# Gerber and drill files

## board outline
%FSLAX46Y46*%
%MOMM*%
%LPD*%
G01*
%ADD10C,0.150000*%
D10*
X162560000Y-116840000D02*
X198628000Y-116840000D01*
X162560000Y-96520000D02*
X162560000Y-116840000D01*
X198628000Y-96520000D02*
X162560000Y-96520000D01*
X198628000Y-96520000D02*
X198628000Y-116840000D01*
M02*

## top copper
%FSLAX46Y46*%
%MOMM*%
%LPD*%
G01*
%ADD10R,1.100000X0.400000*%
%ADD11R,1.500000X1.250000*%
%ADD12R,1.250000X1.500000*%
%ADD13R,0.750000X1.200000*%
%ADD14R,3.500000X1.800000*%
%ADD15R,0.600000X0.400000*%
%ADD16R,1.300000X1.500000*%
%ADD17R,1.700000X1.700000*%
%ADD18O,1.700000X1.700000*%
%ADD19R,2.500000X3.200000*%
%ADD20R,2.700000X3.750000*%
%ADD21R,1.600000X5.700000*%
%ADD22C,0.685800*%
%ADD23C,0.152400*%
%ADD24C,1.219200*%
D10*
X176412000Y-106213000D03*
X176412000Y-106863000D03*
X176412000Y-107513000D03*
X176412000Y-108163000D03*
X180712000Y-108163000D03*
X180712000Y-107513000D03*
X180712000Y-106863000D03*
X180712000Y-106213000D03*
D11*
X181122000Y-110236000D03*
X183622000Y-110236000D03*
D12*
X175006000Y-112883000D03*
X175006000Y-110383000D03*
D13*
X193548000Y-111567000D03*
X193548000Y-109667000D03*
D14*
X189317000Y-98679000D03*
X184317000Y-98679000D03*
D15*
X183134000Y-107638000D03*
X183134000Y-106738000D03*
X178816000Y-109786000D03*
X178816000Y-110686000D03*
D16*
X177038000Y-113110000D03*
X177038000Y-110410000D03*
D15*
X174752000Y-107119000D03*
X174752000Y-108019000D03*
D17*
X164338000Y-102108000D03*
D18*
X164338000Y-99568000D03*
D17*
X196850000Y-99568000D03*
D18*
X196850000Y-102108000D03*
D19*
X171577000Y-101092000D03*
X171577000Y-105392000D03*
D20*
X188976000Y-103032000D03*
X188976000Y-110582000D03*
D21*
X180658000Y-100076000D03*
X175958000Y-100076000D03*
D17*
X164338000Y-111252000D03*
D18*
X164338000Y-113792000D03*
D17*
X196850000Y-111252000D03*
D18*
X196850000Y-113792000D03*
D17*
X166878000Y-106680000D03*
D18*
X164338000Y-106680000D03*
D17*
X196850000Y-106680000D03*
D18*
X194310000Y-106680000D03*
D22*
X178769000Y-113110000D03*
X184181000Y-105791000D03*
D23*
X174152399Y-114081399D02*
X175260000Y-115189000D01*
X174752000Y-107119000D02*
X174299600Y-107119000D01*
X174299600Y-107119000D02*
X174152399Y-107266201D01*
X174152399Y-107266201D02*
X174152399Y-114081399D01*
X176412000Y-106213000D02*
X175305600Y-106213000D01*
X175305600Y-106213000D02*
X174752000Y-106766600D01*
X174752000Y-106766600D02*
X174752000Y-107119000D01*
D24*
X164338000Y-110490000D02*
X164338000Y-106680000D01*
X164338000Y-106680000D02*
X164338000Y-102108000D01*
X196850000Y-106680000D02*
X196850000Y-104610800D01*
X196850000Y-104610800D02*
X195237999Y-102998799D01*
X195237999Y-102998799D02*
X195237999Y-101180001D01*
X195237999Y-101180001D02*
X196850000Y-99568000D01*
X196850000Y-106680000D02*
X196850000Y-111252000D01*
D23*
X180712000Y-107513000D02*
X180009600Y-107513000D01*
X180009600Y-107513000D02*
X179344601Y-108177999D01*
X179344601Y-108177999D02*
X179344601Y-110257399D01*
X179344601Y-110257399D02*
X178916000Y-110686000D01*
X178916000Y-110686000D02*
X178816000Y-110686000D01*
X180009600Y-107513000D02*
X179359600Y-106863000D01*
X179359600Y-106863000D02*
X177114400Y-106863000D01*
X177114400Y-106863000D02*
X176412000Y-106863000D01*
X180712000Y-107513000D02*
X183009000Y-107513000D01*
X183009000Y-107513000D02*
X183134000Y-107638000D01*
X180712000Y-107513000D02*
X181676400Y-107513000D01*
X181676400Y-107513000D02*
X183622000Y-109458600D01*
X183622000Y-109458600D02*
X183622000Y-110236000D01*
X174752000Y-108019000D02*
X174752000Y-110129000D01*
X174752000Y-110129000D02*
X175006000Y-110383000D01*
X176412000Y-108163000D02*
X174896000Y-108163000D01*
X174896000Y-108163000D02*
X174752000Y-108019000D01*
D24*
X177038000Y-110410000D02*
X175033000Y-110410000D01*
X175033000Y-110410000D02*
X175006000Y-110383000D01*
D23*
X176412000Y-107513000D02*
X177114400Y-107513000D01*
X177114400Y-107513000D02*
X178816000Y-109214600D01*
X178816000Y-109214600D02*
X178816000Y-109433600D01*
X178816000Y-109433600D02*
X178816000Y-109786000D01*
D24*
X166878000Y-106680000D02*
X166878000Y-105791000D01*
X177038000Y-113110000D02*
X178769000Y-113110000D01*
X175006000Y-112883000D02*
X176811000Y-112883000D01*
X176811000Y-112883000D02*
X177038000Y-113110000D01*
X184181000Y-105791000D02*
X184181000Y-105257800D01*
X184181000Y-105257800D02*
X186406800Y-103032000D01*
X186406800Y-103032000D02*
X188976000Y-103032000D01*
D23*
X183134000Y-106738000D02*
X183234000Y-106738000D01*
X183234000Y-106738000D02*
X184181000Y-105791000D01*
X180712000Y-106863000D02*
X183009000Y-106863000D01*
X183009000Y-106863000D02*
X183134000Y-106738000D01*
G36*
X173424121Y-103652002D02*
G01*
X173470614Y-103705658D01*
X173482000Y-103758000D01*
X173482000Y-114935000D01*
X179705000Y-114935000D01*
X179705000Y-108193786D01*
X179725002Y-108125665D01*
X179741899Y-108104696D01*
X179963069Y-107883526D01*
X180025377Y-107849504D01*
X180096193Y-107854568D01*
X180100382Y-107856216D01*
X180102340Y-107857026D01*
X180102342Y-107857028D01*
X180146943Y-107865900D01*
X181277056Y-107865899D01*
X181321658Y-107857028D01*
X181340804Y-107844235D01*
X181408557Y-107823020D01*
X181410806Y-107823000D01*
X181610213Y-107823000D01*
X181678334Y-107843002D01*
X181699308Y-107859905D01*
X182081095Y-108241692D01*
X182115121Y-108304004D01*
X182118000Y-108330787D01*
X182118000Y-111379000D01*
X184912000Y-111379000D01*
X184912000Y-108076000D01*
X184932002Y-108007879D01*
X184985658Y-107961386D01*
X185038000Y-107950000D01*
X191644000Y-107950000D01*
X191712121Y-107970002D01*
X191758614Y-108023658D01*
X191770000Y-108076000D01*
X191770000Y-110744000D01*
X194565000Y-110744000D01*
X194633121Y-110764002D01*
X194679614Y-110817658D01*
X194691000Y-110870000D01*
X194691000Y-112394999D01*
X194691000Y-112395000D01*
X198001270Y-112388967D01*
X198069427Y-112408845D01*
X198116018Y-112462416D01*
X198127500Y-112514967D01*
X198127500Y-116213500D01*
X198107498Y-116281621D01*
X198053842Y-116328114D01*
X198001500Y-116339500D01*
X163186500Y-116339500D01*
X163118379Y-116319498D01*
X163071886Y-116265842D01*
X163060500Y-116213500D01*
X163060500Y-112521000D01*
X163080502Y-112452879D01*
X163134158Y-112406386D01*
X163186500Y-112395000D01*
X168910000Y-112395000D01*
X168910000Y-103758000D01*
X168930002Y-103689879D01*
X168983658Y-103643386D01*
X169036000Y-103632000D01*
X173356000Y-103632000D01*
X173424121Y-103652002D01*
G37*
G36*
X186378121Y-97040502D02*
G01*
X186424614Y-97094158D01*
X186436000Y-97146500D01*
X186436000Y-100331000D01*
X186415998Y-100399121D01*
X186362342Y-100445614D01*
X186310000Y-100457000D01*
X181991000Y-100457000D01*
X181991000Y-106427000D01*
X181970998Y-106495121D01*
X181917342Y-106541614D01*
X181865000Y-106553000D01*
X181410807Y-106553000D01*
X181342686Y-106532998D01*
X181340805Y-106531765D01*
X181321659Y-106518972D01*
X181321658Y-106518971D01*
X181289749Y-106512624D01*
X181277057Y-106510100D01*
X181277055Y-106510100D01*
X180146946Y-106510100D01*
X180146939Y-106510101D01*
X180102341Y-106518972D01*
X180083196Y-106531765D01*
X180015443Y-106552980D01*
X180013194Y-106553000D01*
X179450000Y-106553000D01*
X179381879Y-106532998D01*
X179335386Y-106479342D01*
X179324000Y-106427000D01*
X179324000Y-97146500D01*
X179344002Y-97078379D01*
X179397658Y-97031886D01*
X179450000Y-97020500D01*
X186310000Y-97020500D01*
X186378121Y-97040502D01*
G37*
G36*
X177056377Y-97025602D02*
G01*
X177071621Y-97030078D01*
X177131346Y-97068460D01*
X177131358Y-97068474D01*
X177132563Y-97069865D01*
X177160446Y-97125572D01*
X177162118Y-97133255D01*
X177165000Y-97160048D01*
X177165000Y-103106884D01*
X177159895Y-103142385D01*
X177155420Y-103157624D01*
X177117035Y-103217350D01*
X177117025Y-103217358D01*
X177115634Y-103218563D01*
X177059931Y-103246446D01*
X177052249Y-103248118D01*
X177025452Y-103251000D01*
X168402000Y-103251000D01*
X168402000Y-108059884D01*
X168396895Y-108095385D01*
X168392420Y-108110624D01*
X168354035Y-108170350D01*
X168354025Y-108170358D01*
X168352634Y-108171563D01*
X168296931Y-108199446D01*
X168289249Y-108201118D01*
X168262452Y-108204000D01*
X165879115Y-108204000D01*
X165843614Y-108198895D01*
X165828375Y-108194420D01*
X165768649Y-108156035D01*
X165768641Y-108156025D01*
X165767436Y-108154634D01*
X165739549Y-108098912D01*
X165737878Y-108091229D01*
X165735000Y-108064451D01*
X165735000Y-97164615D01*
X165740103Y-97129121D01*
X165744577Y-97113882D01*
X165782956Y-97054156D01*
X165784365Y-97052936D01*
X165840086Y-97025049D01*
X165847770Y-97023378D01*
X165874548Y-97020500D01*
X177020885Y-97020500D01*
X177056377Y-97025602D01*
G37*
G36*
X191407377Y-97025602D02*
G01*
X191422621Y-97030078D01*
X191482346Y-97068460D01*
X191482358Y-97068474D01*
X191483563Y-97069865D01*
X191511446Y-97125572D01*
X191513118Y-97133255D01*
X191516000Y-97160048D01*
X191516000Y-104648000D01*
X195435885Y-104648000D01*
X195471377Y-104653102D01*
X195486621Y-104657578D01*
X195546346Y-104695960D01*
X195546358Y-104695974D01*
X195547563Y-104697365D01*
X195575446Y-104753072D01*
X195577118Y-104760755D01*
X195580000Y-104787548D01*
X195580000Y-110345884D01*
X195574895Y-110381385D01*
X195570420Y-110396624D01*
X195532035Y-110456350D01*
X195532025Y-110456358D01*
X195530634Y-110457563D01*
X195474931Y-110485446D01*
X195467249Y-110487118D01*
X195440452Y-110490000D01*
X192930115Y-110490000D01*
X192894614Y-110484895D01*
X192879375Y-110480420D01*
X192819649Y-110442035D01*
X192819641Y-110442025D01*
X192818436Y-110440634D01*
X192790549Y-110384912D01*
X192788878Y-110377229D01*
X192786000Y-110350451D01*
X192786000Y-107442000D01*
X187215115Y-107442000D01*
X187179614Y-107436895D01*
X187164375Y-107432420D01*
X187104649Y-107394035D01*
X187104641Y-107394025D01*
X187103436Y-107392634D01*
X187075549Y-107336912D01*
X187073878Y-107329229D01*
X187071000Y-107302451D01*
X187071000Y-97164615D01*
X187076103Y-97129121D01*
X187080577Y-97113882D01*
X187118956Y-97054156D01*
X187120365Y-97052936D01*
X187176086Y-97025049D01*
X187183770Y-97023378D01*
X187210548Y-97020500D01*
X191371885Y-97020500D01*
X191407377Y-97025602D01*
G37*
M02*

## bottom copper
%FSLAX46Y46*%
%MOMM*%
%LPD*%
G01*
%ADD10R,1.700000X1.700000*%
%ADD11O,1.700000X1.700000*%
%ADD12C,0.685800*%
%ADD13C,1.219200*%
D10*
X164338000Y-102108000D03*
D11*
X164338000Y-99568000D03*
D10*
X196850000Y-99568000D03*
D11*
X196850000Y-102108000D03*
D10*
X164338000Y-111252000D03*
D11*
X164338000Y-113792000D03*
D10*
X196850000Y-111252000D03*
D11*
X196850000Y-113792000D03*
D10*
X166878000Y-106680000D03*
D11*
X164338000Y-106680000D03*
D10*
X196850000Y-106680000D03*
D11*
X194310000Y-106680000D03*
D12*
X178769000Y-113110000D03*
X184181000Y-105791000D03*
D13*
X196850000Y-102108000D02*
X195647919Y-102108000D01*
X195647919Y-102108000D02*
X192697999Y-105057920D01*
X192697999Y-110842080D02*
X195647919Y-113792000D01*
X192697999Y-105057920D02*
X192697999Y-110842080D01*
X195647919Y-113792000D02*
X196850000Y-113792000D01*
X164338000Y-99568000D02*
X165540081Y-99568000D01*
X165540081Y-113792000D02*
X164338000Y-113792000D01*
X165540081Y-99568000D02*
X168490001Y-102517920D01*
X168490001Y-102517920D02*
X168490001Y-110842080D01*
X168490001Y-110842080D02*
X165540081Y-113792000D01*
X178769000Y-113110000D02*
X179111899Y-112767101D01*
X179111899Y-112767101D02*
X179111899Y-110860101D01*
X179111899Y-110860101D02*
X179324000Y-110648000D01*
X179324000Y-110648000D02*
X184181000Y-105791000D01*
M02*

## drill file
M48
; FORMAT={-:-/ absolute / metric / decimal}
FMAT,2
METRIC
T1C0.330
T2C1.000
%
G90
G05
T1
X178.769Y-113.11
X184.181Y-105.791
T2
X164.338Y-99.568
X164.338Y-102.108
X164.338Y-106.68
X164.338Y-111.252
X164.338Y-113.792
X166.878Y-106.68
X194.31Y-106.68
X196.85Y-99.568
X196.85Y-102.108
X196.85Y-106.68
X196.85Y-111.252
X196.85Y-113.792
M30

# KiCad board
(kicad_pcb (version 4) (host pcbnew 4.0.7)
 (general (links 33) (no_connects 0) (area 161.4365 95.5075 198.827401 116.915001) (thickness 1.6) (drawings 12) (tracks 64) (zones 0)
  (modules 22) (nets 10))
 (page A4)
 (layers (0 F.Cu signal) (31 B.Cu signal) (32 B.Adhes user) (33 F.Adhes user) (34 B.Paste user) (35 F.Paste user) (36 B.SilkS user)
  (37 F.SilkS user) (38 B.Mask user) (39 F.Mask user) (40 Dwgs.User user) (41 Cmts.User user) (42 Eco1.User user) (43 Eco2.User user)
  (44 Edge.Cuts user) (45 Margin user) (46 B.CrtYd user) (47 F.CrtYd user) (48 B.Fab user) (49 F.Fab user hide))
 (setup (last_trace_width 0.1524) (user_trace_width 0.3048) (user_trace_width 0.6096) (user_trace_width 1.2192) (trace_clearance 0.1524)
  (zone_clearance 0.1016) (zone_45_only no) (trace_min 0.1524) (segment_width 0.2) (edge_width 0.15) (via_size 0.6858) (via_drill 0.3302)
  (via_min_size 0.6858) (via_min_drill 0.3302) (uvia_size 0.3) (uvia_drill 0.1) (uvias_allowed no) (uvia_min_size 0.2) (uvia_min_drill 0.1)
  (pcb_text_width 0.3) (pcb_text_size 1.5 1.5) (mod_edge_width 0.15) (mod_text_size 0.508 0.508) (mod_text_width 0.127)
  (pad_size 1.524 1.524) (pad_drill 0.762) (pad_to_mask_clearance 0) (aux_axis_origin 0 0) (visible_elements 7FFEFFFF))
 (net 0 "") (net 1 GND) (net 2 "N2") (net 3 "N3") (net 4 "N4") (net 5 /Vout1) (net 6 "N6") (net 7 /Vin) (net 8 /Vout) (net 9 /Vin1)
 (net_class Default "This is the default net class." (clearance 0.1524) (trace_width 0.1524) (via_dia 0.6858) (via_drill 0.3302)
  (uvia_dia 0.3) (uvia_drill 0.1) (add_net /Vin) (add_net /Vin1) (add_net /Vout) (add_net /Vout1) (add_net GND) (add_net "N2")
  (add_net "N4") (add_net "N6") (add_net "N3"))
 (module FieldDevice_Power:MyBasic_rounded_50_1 (layer B.Cu) (at 180.848 100.457 180)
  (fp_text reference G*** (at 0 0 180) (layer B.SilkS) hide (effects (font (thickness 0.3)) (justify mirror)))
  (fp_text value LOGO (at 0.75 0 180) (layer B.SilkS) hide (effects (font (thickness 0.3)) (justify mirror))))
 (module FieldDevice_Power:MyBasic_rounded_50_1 (layer F.Cu) (at 170.18 111.633)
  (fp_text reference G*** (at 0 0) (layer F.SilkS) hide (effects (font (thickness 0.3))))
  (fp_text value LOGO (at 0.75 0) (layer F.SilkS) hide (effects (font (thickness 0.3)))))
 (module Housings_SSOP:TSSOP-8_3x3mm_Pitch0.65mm (layer F.Cu) (at 178.562 107.188)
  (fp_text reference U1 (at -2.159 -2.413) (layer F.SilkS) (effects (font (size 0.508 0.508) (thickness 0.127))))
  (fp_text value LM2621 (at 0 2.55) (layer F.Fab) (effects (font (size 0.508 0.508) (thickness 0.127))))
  (pad 1 smd rect (at -2.15 -0.975) (size 1.1 0.4) (layers F.Cu F.Paste F.Mask) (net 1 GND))
  (pad 2 smd rect (at -2.15 -0.325) (size 1.1 0.4) (layers F.Cu F.Paste F.Mask) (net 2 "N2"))
  (pad 3 smd rect (at -2.15 0.325) (size 1.1 0.4) (layers F.Cu F.Paste F.Mask) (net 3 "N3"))
  (pad 4 smd rect (at -2.15 0.975) (size 1.1 0.4) (layers F.Cu F.Paste F.Mask) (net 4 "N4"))
  (pad 5 smd rect (at 2.15 0.975) (size 1.1 0.4) (layers F.Cu F.Paste F.Mask) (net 1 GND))
  (pad 6 smd rect (at 2.15 0.325) (size 1.1 0.4) (layers F.Cu F.Paste F.Mask) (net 2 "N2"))
  (pad 7 smd rect (at 2.15 -0.325) (size 1.1 0.4) (layers F.Cu F.Paste F.Mask) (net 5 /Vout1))
  (pad 8 smd rect (at 2.15 -0.975) (size 1.1 0.4) (layers F.Cu F.Paste F.Mask) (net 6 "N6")))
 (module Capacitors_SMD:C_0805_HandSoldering (layer F.Cu) (at 182.372 110.236)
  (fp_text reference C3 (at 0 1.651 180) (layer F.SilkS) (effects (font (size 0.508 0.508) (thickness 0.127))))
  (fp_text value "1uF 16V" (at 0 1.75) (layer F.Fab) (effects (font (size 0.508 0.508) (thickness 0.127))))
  (pad 1 smd rect (at -1.25 0) (size 1.5 1.25) (layers F.Cu F.Paste F.Mask) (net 1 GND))
  (pad 2 smd rect (at 1.25 0) (size 1.5 1.25) (layers F.Cu F.Paste F.Mask) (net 2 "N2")))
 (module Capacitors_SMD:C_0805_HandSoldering (layer F.Cu) (at 175.006 111.633 90)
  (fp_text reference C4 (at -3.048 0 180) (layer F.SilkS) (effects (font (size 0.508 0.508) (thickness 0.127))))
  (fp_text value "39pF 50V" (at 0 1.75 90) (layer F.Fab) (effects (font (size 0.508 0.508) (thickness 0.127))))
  (pad 1 smd rect (at -1.25 0 90) (size 1.5 1.25) (layers F.Cu F.Paste F.Mask) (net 5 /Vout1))
  (pad 2 smd rect (at 1.25 0 90) (size 1.5 1.25) (layers F.Cu F.Paste F.Mask) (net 4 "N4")))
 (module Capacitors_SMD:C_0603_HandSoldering (layer F.Cu) (at 193.548 110.617 90)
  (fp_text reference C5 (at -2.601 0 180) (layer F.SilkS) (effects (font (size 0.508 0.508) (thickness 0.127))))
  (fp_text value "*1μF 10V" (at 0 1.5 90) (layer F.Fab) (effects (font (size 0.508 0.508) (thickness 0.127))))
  (pad 1 smd rect (at -0.95 0 90) (size 1.2 0.75) (layers F.Cu F.Paste F.Mask) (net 1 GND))
  (pad 2 smd rect (at 0.95 0 90) (size 1.2 0.75) (layers F.Cu F.Paste F.Mask) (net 5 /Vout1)))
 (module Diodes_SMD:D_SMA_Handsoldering (layer F.Cu) (at 186.817 98.679 180)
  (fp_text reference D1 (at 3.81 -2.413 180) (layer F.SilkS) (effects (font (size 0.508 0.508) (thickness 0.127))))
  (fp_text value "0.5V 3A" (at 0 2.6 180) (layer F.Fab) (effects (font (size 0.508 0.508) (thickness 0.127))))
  (pad 1 smd rect (at -2.5 0 180) (size 3.5 1.8) (layers F.Cu F.Paste F.Mask) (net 5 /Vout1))
  (pad 2 smd rect (at 2.5 0 180) (size 3.5 1.8) (layers F.Cu F.Paste F.Mask) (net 6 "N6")))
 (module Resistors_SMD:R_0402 (layer F.Cu) (at 183.134 107.188 90)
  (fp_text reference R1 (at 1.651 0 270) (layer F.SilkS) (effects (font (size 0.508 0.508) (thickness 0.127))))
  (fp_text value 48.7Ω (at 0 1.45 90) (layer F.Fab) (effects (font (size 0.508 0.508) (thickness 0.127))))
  (pad 1 smd rect (at -0.45 0 90) (size 0.4 0.6) (layers F.Cu F.Paste F.Mask) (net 2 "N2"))
  (pad 2 smd rect (at 0.45 0 90) (size 0.4 0.6) (layers F.Cu F.Paste F.Mask) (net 5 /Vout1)))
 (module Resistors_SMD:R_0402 (layer F.Cu) (at 178.816 110.236 270)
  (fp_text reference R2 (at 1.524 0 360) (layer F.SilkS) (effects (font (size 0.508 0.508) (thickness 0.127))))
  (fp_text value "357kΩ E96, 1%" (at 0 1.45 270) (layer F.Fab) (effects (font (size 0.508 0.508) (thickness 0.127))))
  (pad 1 smd rect (at -0.45 0 270) (size 0.4 0.6) (layers F.Cu F.Paste F.Mask) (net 3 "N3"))
  (pad 2 smd rect (at 0.45 0 270) (size 0.4 0.6) (layers F.Cu F.Paste F.Mask) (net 2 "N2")))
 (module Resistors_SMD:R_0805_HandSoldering (layer F.Cu) (at 177.038 111.76 90)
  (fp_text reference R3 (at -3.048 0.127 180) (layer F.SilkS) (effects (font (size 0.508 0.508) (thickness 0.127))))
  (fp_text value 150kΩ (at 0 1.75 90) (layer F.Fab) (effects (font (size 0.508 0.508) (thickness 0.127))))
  (pad 1 smd rect (at -1.35 0 90) (size 1.5 1.3) (layers F.Cu F.Paste F.Mask) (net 5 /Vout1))
  (pad 2 smd rect (at 1.35 0 90) (size 1.5 1.3) (layers F.Cu F.Paste F.Mask) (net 4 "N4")))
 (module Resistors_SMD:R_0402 (layer F.Cu) (at 174.752 107.569 270)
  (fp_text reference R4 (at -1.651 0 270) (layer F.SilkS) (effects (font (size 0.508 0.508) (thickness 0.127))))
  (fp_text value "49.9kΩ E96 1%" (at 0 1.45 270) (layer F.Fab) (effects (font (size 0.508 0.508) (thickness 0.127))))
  (pad 1 smd rect (at -0.45 0 270) (size 0.4 0.6) (layers F.Cu F.Paste F.Mask) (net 1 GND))
  (pad 2 smd rect (at 0.45 0 270) (size 0.4 0.6) (layers F.Cu F.Paste F.Mask) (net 4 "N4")))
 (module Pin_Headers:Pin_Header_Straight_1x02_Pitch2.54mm (layer F.Cu) (at 164.338 102.108 180)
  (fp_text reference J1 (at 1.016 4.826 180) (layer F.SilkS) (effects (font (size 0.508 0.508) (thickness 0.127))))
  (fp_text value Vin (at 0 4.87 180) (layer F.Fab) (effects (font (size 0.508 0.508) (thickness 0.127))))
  (pad 1 thru_hole rect (at 0 0 180) (size 1.7 1.7) (drill 1) (layers *.Cu *.Mask) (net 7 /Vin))
  (pad 2 thru_hole oval (at 0 2.54 180) (size 1.7 1.7) (drill 1) (layers *.Cu *.Mask) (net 1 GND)))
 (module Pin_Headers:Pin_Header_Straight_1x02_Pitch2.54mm (layer F.Cu) (at 196.85 99.568)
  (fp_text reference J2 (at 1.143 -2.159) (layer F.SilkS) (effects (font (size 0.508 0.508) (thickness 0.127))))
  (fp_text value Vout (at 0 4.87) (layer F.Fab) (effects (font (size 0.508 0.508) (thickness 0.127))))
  (pad 1 thru_hole rect (at 0 0) (size 1.7 1.7) (drill 1) (layers *.Cu *.Mask) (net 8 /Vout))
  (pad 2 thru_hole oval (at 0 2.54) (size 1.7 1.7) (drill 1) (layers *.Cu *.Mask) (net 1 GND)))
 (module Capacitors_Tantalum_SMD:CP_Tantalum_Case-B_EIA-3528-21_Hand (layer F.Cu) (at 171.577 103.242 270)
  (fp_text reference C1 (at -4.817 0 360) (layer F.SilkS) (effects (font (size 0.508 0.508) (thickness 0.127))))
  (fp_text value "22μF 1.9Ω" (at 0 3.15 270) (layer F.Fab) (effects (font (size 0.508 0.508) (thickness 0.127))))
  (pad 1 smd rect (at -2.15 0 270) (size 3.2 2.5) (layers F.Cu F.Paste F.Mask) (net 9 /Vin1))
  (pad 2 smd rect (at 2.15 0 270) (size 3.2 2.5) (layers F.Cu F.Paste F.Mask) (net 1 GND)))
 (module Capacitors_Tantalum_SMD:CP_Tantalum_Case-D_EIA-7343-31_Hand (layer F.Cu) (at 188.976 106.807 270)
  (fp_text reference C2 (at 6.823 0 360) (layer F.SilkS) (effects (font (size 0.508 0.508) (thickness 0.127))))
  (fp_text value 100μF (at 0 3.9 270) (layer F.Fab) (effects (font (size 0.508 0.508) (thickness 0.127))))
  (pad 1 smd rect (at -3.775 0 270) (size 3.75 2.7) (layers F.Cu F.Paste F.Mask) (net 5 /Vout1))
  (pad 2 smd rect (at 3.775 0 270) (size 3.75 2.7) (layers F.Cu F.Paste F.Mask) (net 1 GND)))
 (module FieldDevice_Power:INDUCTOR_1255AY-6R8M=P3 (layer F.Cu) (at 178.308 100.076)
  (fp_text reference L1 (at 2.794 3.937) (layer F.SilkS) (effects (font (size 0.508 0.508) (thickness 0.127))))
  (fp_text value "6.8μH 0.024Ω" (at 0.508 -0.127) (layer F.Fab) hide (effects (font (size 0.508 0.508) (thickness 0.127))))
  (pad 2 smd rect (at 2.35 0) (size 1.6 5.7) (layers F.Cu F.Paste F.Mask) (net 6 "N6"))
  (pad 1 smd rect (at -2.35 0) (size 1.6 5.7) (layers F.Cu F.Paste F.Mask) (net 9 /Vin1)))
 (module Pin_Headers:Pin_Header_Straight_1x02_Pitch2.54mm (layer F.Cu) (at 164.338 111.252)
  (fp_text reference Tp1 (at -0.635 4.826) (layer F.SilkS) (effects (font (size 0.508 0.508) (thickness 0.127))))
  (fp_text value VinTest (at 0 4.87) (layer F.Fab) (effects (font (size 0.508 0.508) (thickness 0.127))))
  (pad 1 thru_hole rect (at 0 0) (size 1.7 1.7) (drill 1) (layers *.Cu *.Mask) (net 7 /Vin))
  (pad 2 thru_hole oval (at 0 2.54) (size 1.7 1.7) (drill 1) (layers *.Cu *.Mask) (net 1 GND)))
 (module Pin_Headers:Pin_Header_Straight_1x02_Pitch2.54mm (layer F.Cu) (at 196.85 111.252)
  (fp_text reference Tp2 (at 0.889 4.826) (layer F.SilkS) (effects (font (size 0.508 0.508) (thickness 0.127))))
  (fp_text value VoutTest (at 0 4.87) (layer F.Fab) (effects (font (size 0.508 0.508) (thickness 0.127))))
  (pad 1 thru_hole rect (at 0 0) (size 1.7 1.7) (drill 1) (layers *.Cu *.Mask) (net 8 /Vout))
  (pad 2 thru_hole oval (at 0 2.54) (size 1.7 1.7) (drill 1) (layers *.Cu *.Mask) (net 1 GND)))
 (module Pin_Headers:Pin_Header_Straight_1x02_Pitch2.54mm (layer F.Cu) (at 166.878 106.68 270)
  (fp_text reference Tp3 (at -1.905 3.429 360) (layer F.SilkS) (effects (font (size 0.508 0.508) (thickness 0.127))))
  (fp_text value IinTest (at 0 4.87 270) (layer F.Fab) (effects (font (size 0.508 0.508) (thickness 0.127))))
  (pad 1 thru_hole rect (at 0 0 270) (size 1.7 1.7) (drill 1) (layers *.Cu *.Mask) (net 9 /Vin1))
  (pad 2 thru_hole oval (at 0 2.54 270) (size 1.7 1.7) (drill 1) (layers *.Cu *.Mask) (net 7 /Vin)))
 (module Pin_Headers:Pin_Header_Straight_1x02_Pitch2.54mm (layer F.Cu) (at 196.85 106.68 270)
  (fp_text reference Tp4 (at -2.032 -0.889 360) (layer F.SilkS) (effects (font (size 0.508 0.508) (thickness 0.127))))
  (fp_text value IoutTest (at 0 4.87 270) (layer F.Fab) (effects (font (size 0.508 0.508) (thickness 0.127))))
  (pad 1 thru_hole rect (at 0 0 270) (size 1.7 1.7) (drill 1) (layers *.Cu *.Mask) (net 8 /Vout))
  (pad 2 thru_hole oval (at 0 2.54 270) (size 1.7 1.7) (drill 1) (layers *.Cu *.Mask) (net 5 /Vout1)))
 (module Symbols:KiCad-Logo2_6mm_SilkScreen (layer B.Cu) (at 180.848 113.411 180)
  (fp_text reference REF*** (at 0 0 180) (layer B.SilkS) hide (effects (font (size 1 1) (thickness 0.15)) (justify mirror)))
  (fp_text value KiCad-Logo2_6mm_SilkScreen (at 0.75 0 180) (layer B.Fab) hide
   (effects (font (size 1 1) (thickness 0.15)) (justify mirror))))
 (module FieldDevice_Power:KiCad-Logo (layer F.Cu) (at 187.579 114.681)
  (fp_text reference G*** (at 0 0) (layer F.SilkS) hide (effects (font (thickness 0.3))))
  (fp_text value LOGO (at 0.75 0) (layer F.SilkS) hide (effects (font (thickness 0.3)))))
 (gr_line (start 162.56 116.84) (end 198.628 116.84) (layer Edge.Cuts) (width 0.15))
 (gr_line (start 162.56 96.52) (end 162.56 116.84) (layer Edge.Cuts) (width 0.15))
 (gr_line (start 198.628 96.52) (end 162.56 96.52) (layer Edge.Cuts) (width 0.15))
 (gr_line (start 198.628 96.52) (end 198.628 116.84) (layer Edge.Cuts) (width 0.15))
 (segment (start 196.85 102.108) (end 195.647919 102.108) (width 1.2192) (layer B.Cu) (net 1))
 (segment (start 195.647919 102.108) (end 192.697999 105.05792) (width 1.2192) (layer B.Cu) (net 1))
 (segment (start 192.697999 110.84208) (end 195.647919 113.792) (width 1.2192) (layer B.Cu) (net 1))
 (segment (start 192.697999 105.05792) (end 192.697999 110.84208) (width 1.2192) (layer B.Cu) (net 1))
 (segment (start 195.647919 113.792) (end 196.85 113.792) (width 1.2192) (layer B.Cu) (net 1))
 (segment (start 164.338 99.568) (end 165.540081 99.568) (width 1.2192) (layer B.Cu) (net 1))
 (segment (start 165.540081 113.792) (end 164.338 113.792) (width 1.2192) (layer B.Cu) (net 1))
 (segment (start 165.540081 99.568) (end 168.490001 102.51792) (width 1.2192) (layer B.Cu) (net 1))
 (segment (start 168.490001 102.51792) (end 168.490001 110.84208) (width 1.2192) (layer B.Cu) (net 1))
 (segment (start 168.490001 110.84208) (end 165.540081 113.792) (width 1.2192) (layer B.Cu) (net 1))
 (segment (start 174.152399 114.081399) (end 175.26 115.189) (width 0.1524) (layer F.Cu) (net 1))
 (segment (start 174.752 107.119) (end 174.2996 107.119) (width 0.1524) (layer F.Cu) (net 1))
 (segment (start 174.2996 107.119) (end 174.152399 107.266201) (width 0.1524) (layer F.Cu) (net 1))
 (segment (start 174.152399 107.266201) (end 174.152399 114.081399) (width 0.1524) (layer F.Cu) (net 1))
 (segment (start 176.412 106.213) (end 175.3056 106.213) (width 0.1524) (layer F.Cu) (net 1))
 (segment (start 175.3056 106.213) (end 174.752 106.7666) (width 0.1524) (layer F.Cu) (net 1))
 (segment (start 174.752 106.7666) (end 174.752 107.119) (width 0.1524) (layer F.Cu) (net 1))
 (segment (start 164.338 110.49) (end 164.338 106.68) (width 1.2192) (layer F.Cu) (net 7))
 (segment (start 164.338 106.68) (end 164.338 102.108) (width 1.2192) (layer F.Cu) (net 7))
 (segment (start 196.85 106.68) (end 196.85 104.6108) (width 1.2192) (layer F.Cu) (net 8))
 (segment (start 196.85 104.6108) (end 195.237999 102.998799) (width 1.2192) (layer F.Cu) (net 8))
 (segment (start 195.237999 102.998799) (end 195.237999 101.180001) (width 1.2192) (layer F.Cu) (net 8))
 (segment (start 195.237999 101.180001) (end 196.85 99.568) (width 1.2192) (layer F.Cu) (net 8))
 (segment (start 196.85 106.68) (end 196.85 111.252) (width 1.2192) (layer F.Cu) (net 8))
 (segment (start 180.712 107.513) (end 180.0096 107.513) (width 0.1524) (layer F.Cu) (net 2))
 (segment (start 180.0096 107.513) (end 179.344601 108.177999) (width 0.1524) (layer F.Cu) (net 2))
 (segment (start 179.344601 108.177999) (end 179.344601 110.257399) (width 0.1524) (layer F.Cu) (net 2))
 (segment (start 179.344601 110.257399) (end 178.916 110.686) (width 0.1524) (layer F.Cu) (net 2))
 (segment (start 178.916 110.686) (end 178.816 110.686) (width 0.1524) (layer F.Cu) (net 2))
 (segment (start 180.0096 107.513) (end 179.3596 106.863) (width 0.1524) (layer F.Cu) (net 2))
 (segment (start 179.3596 106.863) (end 177.1144 106.863) (width 0.1524) (layer F.Cu) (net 2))
 (segment (start 177.1144 106.863) (end 176.412 106.863) (width 0.1524) (layer F.Cu) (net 2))
 (segment (start 180.712 107.513) (end 183.009 107.513) (width 0.1524) (layer F.Cu) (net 2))
 (segment (start 183.009 107.513) (end 183.134 107.638) (width 0.1524) (layer F.Cu) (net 2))
 (segment (start 180.712 107.513) (end 181.6764 107.513) (width 0.1524) (layer F.Cu) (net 2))
 (segment (start 181.6764 107.513) (end 183.622 109.4586) (width 0.1524) (layer F.Cu) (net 2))
 (segment (start 183.622 109.4586) (end 183.622 110.236) (width 0.1524) (layer F.Cu) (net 2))
 (segment (start 174.752 108.019) (end 174.752 110.129) (width 0.1524) (layer F.Cu) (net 4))
 (segment (start 174.752 110.129) (end 175.006 110.383) (width 0.1524) (layer F.Cu) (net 4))
 (segment (start 176.412 108.163) (end 174.896 108.163) (width 0.1524) (layer F.Cu) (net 4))
 (segment (start 174.896 108.163) (end 174.752 108.019) (width 0.1524) (layer F.Cu) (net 4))
 (segment (start 177.038 110.41) (end 175.033 110.41) (width 1.2192) (layer F.Cu) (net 4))
 (segment (start 175.033 110.41) (end 175.006 110.383) (width 1.2192) (layer F.Cu) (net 4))
 (segment (start 176.412 107.513) (end 177.1144 107.513) (width 0.1524) (layer F.Cu) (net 3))
 (segment (start 177.1144 107.513) (end 178.816 109.2146) (width 0.1524) (layer F.Cu) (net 3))
 (segment (start 178.816 109.2146) (end 178.816 109.4336) (width 0.1524) (layer F.Cu) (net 3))
 (segment (start 178.816 109.4336) (end 178.816 109.786) (width 0.1524) (layer F.Cu) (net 3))
 (segment (start 166.878 106.68) (end 166.878 105.791) (width 1.2192) (layer F.Cu) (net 9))
 (segment (start 178.769 113.11) (end 179.111899 112.767101) (width 1.2192) (layer B.Cu) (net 5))
 (segment (start 179.111899 112.767101) (end 179.111899 110.860101) (width 1.2192) (layer B.Cu) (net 5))
 (segment (start 179.111899 110.860101) (end 179.324 110.648) (width 1.2192) (layer B.Cu) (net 5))
 (via (at 178.769 113.11) (size 0.6858) (drill 0.3302) (layers F.Cu B.Cu) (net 5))
 (segment (start 177.038 113.11) (end 178.769 113.11) (width 1.2192) (layer F.Cu) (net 5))
 (segment (start 179.324 110.648) (end 184.181 105.791) (width 1.2192) (layer B.Cu) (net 5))
 (via (at 184.181 105.791) (size 0.6858) (drill 0.3302) (layers F.Cu B.Cu) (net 5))
 (segment (start 175.006 112.883) (end 176.811 112.883) (width 1.2192) (layer F.Cu) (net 5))
 (segment (start 176.811 112.883) (end 177.038 113.11) (width 1.2192) (layer F.Cu) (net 5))
 (segment (start 184.181 105.791) (end 184.181 105.2578) (width 1.2192) (layer F.Cu) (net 5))
 (segment (start 184.181 105.2578) (end 186.4068 103.032) (width 1.2192) (layer F.Cu) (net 5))
 (segment (start 186.4068 103.032) (end 188.976 103.032) (width 1.2192) (layer F.Cu) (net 5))
 (segment (start 183.134 106.738) (end 183.234 106.738) (width 0.1524) (layer F.Cu) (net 5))
 (segment (start 183.234 106.738) (end 184.181 105.791) (width 0.1524) (layer F.Cu) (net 5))
 (segment (start 180.712 106.863) (end 183.009 106.863) (width 0.1524) (layer F.Cu) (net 5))
 (segment (start 183.009 106.863) (end 183.134 106.738) (width 0.1524) (layer F.Cu) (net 5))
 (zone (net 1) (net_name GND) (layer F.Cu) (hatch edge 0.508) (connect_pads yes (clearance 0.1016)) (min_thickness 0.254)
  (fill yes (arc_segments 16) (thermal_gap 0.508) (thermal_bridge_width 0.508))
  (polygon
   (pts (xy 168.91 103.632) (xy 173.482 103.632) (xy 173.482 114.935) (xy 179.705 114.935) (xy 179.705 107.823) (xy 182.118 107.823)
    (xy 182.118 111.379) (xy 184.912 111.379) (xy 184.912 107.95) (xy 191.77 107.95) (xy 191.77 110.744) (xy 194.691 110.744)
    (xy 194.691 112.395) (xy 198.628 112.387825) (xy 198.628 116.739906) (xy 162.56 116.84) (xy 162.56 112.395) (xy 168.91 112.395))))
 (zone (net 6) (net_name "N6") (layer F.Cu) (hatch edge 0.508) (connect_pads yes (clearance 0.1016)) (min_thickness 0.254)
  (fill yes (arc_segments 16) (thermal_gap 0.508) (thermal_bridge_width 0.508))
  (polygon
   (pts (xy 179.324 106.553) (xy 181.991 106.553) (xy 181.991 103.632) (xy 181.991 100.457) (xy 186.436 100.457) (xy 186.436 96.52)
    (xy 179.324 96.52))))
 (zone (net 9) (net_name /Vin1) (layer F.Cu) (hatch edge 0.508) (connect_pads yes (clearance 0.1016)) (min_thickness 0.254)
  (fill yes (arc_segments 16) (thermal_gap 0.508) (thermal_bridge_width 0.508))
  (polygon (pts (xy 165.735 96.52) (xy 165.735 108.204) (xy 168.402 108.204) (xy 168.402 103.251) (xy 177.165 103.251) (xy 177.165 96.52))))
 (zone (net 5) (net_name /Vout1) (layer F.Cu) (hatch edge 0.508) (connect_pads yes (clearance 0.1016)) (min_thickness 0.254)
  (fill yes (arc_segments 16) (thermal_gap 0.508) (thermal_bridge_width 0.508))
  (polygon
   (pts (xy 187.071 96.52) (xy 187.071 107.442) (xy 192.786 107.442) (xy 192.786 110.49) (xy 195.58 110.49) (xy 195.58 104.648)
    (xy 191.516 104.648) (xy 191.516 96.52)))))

